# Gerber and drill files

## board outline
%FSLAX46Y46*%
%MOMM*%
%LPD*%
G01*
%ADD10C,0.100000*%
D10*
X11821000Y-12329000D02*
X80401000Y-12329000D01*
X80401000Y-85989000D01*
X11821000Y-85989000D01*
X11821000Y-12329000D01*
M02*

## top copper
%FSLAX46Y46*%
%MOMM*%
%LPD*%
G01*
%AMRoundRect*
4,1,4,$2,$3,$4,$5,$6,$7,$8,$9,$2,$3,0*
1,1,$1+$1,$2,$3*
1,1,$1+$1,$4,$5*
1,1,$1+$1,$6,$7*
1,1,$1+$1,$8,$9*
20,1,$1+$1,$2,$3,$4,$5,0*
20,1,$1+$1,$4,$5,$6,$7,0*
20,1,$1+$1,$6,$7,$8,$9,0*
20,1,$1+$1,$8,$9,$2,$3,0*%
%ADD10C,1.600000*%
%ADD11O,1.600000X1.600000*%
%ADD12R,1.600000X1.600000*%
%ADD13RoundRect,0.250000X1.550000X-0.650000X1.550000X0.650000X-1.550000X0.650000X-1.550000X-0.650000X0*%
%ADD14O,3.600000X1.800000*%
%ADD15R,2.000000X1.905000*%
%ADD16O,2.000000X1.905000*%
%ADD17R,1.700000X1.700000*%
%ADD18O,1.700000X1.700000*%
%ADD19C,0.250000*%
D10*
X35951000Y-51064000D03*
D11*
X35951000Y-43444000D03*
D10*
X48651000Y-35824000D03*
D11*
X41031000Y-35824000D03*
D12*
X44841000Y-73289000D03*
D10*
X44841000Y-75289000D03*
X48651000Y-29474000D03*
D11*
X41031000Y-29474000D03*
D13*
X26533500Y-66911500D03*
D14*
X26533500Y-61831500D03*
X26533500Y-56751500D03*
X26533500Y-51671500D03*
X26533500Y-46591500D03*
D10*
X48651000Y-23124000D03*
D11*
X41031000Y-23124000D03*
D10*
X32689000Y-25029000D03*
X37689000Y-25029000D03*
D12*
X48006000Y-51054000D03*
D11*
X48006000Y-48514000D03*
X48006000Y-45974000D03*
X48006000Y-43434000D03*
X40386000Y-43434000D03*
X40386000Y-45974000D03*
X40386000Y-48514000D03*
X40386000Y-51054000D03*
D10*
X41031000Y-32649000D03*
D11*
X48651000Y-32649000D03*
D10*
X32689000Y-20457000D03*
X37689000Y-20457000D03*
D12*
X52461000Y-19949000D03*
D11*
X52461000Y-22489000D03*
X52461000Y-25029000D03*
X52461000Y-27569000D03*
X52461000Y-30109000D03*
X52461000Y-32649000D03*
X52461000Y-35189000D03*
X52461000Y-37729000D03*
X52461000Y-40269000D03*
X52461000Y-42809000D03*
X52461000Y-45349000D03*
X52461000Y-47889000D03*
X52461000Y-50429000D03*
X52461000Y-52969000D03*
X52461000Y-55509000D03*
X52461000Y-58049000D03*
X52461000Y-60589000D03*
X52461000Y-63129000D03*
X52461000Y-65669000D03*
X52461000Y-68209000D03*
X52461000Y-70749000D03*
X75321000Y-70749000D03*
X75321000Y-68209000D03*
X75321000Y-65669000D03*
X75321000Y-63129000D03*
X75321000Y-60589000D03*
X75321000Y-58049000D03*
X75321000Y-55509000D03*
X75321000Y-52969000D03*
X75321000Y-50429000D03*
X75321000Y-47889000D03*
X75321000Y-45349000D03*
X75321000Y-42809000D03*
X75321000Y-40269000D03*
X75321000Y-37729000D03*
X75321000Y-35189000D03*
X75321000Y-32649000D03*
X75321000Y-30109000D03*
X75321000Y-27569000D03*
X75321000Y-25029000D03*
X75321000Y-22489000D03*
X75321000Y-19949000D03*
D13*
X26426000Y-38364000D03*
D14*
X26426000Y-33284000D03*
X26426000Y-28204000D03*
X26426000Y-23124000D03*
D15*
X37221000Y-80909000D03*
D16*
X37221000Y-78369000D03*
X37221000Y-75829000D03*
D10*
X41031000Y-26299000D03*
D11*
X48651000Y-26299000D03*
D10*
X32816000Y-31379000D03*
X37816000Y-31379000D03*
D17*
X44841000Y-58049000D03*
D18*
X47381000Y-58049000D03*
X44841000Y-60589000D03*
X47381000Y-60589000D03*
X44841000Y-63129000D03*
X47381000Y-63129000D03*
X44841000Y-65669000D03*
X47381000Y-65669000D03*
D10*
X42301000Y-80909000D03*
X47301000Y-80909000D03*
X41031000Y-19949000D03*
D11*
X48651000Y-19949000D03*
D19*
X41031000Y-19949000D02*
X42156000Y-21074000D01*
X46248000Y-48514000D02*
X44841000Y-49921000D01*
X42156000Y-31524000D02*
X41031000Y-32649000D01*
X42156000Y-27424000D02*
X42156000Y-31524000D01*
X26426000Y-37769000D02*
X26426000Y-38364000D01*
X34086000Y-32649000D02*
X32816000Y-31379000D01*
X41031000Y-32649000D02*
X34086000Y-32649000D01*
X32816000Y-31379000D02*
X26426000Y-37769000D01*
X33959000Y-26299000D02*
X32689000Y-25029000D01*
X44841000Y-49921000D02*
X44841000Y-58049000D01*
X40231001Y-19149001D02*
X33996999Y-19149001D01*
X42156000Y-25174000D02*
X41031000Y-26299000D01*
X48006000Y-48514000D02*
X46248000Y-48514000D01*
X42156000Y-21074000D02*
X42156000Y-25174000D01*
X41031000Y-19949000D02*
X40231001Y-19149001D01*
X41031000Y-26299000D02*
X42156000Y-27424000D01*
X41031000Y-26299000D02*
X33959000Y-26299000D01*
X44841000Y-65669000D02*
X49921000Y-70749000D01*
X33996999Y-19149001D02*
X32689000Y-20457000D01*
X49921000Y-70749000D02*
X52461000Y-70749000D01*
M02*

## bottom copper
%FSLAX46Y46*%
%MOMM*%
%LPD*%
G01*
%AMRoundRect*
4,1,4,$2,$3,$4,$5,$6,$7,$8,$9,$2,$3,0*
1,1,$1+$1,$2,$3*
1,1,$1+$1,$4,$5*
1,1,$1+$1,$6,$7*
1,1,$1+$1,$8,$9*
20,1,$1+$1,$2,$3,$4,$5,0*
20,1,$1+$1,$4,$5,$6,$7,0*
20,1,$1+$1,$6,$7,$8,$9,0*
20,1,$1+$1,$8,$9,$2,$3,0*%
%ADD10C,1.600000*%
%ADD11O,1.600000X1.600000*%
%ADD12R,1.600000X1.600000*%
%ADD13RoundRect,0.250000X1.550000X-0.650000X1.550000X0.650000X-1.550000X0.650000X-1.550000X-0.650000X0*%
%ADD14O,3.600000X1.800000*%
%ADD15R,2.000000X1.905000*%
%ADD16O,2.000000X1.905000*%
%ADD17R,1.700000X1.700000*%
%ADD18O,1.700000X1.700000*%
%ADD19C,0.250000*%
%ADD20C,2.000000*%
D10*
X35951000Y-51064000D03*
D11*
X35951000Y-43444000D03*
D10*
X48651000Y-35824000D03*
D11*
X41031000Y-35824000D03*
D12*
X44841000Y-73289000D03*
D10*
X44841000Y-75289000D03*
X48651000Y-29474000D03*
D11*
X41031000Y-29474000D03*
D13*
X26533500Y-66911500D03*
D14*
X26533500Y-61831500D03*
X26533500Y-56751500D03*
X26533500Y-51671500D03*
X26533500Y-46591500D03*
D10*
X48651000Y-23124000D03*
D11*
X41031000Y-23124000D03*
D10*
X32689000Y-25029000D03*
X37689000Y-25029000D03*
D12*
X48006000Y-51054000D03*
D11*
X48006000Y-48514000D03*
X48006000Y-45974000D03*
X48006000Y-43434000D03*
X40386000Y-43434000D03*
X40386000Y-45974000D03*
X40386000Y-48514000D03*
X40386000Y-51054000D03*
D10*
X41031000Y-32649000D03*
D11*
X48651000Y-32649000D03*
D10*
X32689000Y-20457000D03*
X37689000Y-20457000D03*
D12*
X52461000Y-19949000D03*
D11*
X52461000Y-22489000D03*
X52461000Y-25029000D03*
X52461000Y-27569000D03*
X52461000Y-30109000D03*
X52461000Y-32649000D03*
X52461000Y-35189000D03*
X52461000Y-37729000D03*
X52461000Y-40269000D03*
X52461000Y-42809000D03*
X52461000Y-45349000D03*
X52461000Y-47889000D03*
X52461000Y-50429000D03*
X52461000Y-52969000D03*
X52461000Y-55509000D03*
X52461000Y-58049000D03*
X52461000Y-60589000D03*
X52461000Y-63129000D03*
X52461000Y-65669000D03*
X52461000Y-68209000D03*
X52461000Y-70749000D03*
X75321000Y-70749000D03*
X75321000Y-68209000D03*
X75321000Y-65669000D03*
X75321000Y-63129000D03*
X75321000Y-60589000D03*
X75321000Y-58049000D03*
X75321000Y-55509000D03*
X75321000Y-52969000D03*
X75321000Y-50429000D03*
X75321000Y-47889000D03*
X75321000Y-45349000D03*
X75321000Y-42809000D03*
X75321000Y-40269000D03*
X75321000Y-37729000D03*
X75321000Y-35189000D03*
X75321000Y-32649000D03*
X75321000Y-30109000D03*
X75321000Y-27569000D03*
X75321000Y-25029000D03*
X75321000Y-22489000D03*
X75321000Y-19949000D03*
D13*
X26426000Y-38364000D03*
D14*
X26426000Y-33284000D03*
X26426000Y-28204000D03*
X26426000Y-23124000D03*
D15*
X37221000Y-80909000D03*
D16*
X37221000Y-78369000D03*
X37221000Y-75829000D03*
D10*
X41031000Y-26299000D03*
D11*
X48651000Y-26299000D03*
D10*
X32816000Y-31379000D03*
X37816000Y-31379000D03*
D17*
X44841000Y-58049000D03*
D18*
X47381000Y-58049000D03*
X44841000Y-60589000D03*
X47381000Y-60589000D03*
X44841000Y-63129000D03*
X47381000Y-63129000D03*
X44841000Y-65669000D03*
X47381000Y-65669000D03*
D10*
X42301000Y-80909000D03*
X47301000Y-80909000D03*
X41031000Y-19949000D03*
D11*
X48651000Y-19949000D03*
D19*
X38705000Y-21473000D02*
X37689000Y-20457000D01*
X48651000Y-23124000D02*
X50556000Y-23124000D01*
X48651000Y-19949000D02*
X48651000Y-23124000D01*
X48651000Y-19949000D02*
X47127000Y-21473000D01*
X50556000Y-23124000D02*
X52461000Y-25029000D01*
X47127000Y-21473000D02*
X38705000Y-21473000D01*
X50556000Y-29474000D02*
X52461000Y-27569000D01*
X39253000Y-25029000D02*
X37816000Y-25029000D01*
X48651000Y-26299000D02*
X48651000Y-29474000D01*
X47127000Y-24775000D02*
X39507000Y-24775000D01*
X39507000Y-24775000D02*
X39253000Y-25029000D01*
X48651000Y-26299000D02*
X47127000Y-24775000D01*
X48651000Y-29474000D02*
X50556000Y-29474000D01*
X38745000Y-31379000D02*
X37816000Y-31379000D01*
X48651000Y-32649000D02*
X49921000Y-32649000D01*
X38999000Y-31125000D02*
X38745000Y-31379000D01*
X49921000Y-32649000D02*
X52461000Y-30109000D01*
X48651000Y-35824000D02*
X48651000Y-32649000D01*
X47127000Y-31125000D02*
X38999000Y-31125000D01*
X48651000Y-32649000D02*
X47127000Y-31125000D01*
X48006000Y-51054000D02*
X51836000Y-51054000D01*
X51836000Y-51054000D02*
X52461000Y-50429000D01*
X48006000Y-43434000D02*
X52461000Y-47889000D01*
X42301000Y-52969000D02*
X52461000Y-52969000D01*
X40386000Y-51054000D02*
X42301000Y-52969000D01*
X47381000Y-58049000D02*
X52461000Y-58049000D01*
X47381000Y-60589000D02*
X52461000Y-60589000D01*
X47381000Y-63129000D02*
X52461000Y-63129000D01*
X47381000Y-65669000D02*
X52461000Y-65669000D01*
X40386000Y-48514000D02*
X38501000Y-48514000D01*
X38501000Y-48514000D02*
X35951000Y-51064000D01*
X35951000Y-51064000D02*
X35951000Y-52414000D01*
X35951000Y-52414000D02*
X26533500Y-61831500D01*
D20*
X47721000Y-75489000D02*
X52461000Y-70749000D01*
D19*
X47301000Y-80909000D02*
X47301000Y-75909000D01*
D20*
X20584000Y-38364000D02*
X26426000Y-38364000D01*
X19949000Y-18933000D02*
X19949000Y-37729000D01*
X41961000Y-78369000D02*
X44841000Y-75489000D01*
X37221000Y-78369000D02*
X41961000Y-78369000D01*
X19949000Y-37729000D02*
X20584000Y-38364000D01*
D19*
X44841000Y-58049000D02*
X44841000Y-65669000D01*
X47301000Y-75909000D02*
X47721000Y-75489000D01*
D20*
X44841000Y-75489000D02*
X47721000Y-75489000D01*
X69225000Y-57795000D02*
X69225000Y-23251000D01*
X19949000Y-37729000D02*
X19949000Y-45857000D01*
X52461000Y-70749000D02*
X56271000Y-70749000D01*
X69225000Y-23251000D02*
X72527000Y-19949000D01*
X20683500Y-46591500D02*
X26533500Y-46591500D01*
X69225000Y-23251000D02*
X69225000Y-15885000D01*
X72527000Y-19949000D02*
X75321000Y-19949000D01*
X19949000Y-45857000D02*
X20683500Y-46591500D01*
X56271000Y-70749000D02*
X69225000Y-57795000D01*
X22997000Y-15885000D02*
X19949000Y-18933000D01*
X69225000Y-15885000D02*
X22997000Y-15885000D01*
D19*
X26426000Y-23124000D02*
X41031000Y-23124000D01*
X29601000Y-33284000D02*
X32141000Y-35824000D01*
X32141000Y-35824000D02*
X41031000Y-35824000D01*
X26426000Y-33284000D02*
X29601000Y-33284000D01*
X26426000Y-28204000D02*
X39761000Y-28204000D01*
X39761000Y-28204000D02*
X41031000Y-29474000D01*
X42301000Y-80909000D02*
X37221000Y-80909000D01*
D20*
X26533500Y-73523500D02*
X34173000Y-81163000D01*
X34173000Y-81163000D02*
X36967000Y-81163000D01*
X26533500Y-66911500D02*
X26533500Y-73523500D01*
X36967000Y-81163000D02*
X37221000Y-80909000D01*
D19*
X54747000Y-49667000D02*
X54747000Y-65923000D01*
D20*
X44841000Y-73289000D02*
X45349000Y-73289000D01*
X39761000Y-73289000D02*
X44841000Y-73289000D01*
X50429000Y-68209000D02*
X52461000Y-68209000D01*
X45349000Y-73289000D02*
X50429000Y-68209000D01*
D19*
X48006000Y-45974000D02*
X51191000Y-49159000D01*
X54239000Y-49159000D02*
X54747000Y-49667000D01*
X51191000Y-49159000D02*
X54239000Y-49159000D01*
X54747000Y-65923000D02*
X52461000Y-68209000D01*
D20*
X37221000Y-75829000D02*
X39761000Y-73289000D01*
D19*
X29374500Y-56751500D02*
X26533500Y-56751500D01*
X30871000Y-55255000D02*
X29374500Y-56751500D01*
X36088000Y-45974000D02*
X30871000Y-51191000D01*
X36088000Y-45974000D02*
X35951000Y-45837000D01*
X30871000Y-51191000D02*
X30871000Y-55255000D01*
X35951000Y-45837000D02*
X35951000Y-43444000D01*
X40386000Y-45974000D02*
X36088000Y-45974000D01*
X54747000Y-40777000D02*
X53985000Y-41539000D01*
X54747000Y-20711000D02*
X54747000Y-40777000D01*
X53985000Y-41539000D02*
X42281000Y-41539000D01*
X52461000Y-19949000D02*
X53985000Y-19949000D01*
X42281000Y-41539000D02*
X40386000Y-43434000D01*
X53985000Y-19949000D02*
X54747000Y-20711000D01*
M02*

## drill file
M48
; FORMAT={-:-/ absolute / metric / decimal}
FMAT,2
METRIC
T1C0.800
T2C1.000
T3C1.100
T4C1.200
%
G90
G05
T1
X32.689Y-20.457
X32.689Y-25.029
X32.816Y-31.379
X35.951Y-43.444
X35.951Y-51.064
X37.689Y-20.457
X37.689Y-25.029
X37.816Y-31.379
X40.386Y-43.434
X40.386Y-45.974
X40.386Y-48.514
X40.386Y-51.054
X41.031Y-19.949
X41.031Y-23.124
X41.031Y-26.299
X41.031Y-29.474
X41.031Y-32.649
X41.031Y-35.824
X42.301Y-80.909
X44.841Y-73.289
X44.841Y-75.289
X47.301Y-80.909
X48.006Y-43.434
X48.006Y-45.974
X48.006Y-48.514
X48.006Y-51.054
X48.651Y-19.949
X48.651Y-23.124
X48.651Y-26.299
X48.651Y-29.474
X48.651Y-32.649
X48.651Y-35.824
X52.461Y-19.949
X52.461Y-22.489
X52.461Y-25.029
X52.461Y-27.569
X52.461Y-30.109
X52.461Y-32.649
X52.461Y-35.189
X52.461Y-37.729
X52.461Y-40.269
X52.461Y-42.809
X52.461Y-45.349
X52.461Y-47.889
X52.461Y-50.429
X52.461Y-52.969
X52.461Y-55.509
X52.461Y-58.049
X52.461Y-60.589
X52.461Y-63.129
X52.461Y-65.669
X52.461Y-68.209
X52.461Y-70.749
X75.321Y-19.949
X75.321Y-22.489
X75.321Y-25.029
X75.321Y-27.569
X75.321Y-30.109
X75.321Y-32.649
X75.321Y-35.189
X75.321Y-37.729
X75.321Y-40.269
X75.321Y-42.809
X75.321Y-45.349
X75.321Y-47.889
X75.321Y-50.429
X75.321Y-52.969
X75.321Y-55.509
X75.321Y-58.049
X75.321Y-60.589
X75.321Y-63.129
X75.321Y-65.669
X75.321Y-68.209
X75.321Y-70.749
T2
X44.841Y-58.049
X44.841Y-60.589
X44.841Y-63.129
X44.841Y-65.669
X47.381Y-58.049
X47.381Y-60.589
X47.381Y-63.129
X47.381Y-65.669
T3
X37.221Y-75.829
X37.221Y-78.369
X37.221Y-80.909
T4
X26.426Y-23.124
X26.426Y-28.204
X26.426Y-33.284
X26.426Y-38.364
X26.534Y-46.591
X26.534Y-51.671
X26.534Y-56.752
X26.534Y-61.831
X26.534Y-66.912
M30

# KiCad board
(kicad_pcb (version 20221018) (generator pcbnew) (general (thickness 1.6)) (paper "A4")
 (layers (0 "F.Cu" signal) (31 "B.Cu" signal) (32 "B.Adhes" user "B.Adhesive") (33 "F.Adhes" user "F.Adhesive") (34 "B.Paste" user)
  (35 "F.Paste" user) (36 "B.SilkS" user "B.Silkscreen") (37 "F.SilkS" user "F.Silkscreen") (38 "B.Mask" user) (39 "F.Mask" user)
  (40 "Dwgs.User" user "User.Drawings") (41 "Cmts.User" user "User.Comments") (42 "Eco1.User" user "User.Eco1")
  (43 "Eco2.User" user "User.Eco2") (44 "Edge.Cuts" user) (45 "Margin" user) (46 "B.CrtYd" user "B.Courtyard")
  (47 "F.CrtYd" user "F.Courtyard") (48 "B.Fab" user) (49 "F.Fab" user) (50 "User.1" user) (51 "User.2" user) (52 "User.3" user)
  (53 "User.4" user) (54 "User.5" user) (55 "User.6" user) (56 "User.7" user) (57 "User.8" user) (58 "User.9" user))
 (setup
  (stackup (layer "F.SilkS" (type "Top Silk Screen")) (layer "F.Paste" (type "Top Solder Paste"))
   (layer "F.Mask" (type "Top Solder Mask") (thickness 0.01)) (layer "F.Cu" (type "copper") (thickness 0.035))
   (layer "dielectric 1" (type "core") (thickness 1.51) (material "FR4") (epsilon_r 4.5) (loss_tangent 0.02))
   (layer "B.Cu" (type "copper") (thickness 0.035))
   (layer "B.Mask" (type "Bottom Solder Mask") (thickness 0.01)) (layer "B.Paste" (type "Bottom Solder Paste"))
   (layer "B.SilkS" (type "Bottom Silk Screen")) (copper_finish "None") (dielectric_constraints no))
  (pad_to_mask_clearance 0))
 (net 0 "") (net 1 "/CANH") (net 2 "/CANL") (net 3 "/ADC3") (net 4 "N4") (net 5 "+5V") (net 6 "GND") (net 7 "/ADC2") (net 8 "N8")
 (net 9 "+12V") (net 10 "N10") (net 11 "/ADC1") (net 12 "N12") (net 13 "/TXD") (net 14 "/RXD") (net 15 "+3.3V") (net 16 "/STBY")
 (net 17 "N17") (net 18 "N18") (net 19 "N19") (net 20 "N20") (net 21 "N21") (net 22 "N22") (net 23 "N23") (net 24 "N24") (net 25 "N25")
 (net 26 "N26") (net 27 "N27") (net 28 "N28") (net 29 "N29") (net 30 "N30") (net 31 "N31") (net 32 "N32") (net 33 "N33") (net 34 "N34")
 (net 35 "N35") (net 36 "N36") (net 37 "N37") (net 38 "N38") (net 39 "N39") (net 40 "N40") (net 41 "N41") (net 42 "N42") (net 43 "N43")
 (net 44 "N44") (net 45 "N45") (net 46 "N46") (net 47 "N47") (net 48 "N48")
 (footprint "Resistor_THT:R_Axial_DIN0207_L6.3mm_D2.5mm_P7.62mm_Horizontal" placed (layer "F.Cu") (at 35.951 51.064 90)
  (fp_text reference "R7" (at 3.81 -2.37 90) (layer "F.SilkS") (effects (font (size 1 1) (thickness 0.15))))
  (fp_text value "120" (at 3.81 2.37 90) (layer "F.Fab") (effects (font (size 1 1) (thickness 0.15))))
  (pad "1" thru_hole circle (at 0 0 90) (size 1.6 1.6) (drill 0.8) (layers "*.Cu" "*.Mask") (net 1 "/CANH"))
  (pad "2" thru_hole oval (at 7.62 0 90) (size 1.6 1.6) (drill 0.8) (layers "*.Cu" "*.Mask") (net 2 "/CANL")))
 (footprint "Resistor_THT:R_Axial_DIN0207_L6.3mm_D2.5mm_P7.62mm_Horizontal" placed (layer "F.Cu") (at 48.651 35.824 180)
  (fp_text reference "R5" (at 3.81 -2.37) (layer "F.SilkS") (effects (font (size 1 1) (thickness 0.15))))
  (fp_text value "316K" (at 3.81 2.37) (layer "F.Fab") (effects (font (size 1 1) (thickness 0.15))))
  (pad "1" thru_hole circle (at 0 0 180) (size 1.6 1.6) (drill 0.8) (layers "*.Cu" "*.Mask") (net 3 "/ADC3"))
  (pad "2" thru_hole oval (at 7.62 0 180) (size 1.6 1.6) (drill 0.8) (layers "*.Cu" "*.Mask") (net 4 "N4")))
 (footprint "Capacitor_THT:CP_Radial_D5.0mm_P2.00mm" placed (layer "F.Cu") (at 44.841 73.289 -90)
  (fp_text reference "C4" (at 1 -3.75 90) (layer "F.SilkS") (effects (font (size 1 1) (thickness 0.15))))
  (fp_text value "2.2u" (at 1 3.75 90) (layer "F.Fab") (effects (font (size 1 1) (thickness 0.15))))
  (pad "1" thru_hole rect (at 0 0 270) (size 1.6 1.6) (drill 0.8) (layers "*.Cu" "*.Mask") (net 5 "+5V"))
  (pad "2" thru_hole circle (at 2 0 270) (size 1.6 1.6) (drill 0.8) (layers "*.Cu" "*.Mask") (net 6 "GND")))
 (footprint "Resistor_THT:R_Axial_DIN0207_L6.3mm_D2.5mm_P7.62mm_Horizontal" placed (layer "F.Cu") (at 48.651 29.474 180)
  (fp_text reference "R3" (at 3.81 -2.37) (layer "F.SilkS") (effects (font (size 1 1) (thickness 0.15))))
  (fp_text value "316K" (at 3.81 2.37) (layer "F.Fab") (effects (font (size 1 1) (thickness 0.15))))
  (pad "1" thru_hole circle (at 0 0 180) (size 1.6 1.6) (drill 0.8) (layers "*.Cu" "*.Mask") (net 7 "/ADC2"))
  (pad "2" thru_hole oval (at 7.62 0 180) (size 1.6 1.6) (drill 0.8) (layers "*.Cu" "*.Mask") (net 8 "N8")))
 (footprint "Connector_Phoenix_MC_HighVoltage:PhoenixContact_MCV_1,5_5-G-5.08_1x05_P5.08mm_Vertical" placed (layer "F.Cu")
  (at 26.5335 66.9115 90)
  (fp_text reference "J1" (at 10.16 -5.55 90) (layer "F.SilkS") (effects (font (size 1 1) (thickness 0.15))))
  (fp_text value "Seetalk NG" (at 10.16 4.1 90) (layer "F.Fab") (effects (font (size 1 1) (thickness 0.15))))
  (pad "1" thru_hole roundrect (at 0 0 90) (size 1.8 3.6) (drill 1.2) (layers "*.Cu" "*.Mask") (roundrect_rratio 0.138889) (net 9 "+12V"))
  (pad "2" thru_hole oval (at 5.08 0 90) (size 1.8 3.6) (drill 1.2) (layers "*.Cu" "*.Mask") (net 1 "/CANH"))
  (pad "3" thru_hole oval (at 10.16 0 90) (size 1.8 3.6) (drill 1.2) (layers "*.Cu" "*.Mask") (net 2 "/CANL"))
  (pad "4" thru_hole oval (at 15.24 0 90) (size 1.8 3.6) (drill 1.2) (layers "*.Cu" "*.Mask") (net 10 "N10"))
  (pad "5" thru_hole oval (at 20.32 0 90) (size 1.8 3.6) (drill 1.2) (layers "*.Cu" "*.Mask") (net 6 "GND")))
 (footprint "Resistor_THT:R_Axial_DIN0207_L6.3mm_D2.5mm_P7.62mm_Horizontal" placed (layer "F.Cu") (at 48.651 23.124 180)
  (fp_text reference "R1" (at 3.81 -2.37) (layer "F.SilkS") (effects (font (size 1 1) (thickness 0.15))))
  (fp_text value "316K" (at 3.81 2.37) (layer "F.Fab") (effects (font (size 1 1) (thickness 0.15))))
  (pad "1" thru_hole circle (at 0 0 180) (size 1.6 1.6) (drill 0.8) (layers "*.Cu" "*.Mask") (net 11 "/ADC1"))
  (pad "2" thru_hole oval (at 7.62 0 180) (size 1.6 1.6) (drill 0.8) (layers "*.Cu" "*.Mask") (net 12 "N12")))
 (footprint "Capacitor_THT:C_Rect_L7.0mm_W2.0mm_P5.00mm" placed (layer "F.Cu") (at 32.689 25.029)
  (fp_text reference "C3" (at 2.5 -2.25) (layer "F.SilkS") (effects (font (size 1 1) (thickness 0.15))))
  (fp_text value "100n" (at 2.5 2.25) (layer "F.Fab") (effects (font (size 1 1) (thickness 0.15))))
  (pad "1" thru_hole circle (at 0 0) (size 1.6 1.6) (drill 0.8) (layers "*.Cu" "*.Mask") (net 6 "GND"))
  (pad "2" thru_hole circle (at 5 0) (size 1.6 1.6) (drill 0.8) (layers "*.Cu" "*.Mask") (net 7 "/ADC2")))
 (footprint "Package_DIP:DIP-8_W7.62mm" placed (layer "F.Cu") (at 48.006 51.054 180)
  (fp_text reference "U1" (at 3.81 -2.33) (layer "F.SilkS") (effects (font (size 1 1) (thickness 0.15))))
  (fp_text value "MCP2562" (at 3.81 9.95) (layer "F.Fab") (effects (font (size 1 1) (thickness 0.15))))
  (pad "1" thru_hole rect (at 0 0 180) (size 1.6 1.6) (drill 0.8) (layers "*.Cu" "*.Mask") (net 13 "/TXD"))
  (pad "2" thru_hole oval (at 0 2.54 180) (size 1.6 1.6) (drill 0.8) (layers "*.Cu" "*.Mask") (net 6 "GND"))
  (pad "3" thru_hole oval (at 0 5.08 180) (size 1.6 1.6) (drill 0.8) (layers "*.Cu" "*.Mask") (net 5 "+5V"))
  (pad "4" thru_hole oval (at 0 7.62 180) (size 1.6 1.6) (drill 0.8) (layers "*.Cu" "*.Mask") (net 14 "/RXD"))
  (pad "5" thru_hole oval (at 7.62 7.62 180) (size 1.6 1.6) (drill 0.8) (layers "*.Cu" "*.Mask") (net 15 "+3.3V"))
  (pad "6" thru_hole oval (at 7.62 5.08 180) (size 1.6 1.6) (drill 0.8) (layers "*.Cu" "*.Mask") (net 2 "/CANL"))
  (pad "7" thru_hole oval (at 7.62 2.54 180) (size 1.6 1.6) (drill 0.8) (layers "*.Cu" "*.Mask") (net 1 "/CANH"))
  (pad "8" thru_hole oval (at 7.62 0 180) (size 1.6 1.6) (drill 0.8) (layers "*.Cu" "*.Mask") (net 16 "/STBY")))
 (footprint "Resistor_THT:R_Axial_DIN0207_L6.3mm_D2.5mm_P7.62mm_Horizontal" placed (layer "F.Cu") (at 41.031 32.649)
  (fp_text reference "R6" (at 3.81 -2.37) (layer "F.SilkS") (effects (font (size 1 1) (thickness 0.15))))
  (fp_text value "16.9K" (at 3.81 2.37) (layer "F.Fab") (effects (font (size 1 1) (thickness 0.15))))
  (pad "1" thru_hole circle (at 0 0) (size 1.6 1.6) (drill 0.8) (layers "*.Cu" "*.Mask") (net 6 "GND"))
  (pad "2" thru_hole oval (at 7.62 0) (size 1.6 1.6) (drill 0.8) (layers "*.Cu" "*.Mask") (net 3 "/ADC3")))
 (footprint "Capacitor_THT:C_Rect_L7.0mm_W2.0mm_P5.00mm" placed (layer "F.Cu") (at 32.689 20.457)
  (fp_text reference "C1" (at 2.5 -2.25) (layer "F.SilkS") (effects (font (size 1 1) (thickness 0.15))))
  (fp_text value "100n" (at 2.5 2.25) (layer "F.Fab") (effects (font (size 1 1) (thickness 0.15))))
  (pad "1" thru_hole circle (at 0 0) (size 1.6 1.6) (drill 0.8) (layers "*.Cu" "*.Mask") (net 6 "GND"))
  (pad "2" thru_hole circle (at 5 0) (size 1.6 1.6) (drill 0.8) (layers "*.Cu" "*.Mask") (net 11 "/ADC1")))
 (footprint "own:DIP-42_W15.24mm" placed (layer "F.Cu") (at 52.461 19.949)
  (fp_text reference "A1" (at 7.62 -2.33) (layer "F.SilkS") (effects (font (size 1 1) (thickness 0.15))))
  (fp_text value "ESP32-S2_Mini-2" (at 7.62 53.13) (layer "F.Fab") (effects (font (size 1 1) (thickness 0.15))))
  (pad "1" thru_hole rect (at 0 0) (size 1.6 1.6) (drill 0.8) (layers "*.Cu" "*.Mask") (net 15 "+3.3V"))
  (pad "2" thru_hole oval (at 0 2.54) (size 1.6 1.6) (drill 0.8) (layers "*.Cu" "*.Mask") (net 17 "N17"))
  (pad "3" thru_hole oval (at 0 5.08) (size 1.6 1.6) (drill 0.8) (layers "*.Cu" "*.Mask") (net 11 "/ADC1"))
  (pad "4" thru_hole oval (at 0 7.62) (size 1.6 1.6) (drill 0.8) (layers "*.Cu" "*.Mask") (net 7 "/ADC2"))
  (pad "5" thru_hole oval (at 0 10.16) (size 1.6 1.6) (drill 0.8) (layers "*.Cu" "*.Mask") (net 3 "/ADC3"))
  (pad "6" thru_hole oval (at 0 12.7) (size 1.6 1.6) (drill 0.8) (layers "*.Cu" "*.Mask") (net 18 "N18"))
  (pad "7" thru_hole oval (at 0 15.24) (size 1.6 1.6) (drill 0.8) (layers "*.Cu" "*.Mask") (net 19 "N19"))
  (pad "8" thru_hole oval (at 0 17.78) (size 1.6 1.6) (drill 0.8) (layers "*.Cu" "*.Mask") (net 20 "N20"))
  (pad "9" thru_hole oval (at 0 20.32) (size 1.6 1.6) (drill 0.8) (layers "*.Cu" "*.Mask") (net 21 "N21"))
  (pad "10" thru_hole oval (at 0 22.86) (size 1.6 1.6) (drill 0.8) (layers "*.Cu" "*.Mask") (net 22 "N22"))
  (pad "11" thru_hole oval (at 0 25.4) (size 1.6 1.6) (drill 0.8) (layers "*.Cu" "*.Mask") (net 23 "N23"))
  (pad "12" thru_hole oval (at 0 27.94) (size 1.6 1.6) (drill 0.8) (layers "*.Cu" "*.Mask") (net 14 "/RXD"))
  (pad "13" thru_hole oval (at 0 30.48) (size 1.6 1.6) (drill 0.8) (layers "*.Cu" "*.Mask") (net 13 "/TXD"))
  (pad "14" thru_hole oval (at 0 33.02) (size 1.6 1.6) (drill 0.8) (layers "*.Cu" "*.Mask") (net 16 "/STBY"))
  (pad "15" thru_hole oval (at 0 35.56) (size 1.6 1.6) (drill 0.8) (layers "*.Cu" "*.Mask") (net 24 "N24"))
  (pad "16" thru_hole oval (at 0 38.1) (size 1.6 1.6) (drill 0.8) (layers "*.Cu" "*.Mask") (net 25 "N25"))
  (pad "17" thru_hole oval (at 0 40.64) (size 1.6 1.6) (drill 0.8) (layers "*.Cu" "*.Mask") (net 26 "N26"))
  (pad "18" thru_hole oval (at 0 43.18) (size 1.6 1.6) (drill 0.8) (layers "*.Cu" "*.Mask") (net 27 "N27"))
  (pad "19" thru_hole oval (at 0 45.72) (size 1.6 1.6) (drill 0.8) (layers "*.Cu" "*.Mask") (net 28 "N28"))
  (pad "20" thru_hole oval (at 0 48.26) (size 1.6 1.6) (drill 0.8) (layers "*.Cu" "*.Mask") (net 5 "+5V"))
  (pad "21" thru_hole oval (at 0 50.8) (size 1.6 1.6) (drill 0.8) (layers "*.Cu" "*.Mask") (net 6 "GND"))
  (pad "22" thru_hole oval (at 22.86 50.8) (size 1.6 1.6) (drill 0.8) (layers "*.Cu" "*.Mask") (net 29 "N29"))
  (pad "23" thru_hole oval (at 22.86 48.26) (size 1.6 1.6) (drill 0.8) (layers "*.Cu" "*.Mask") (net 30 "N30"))
  (pad "24" thru_hole oval (at 22.86 45.72) (size 1.6 1.6) (drill 0.8) (layers "*.Cu" "*.Mask") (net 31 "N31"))
  (pad "25" thru_hole oval (at 22.86 43.18) (size 1.6 1.6) (drill 0.8) (layers "*.Cu" "*.Mask") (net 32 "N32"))
  (pad "26" thru_hole oval (at 22.86 40.64) (size 1.6 1.6) (drill 0.8) (layers "*.Cu" "*.Mask") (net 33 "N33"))
  (pad "27" thru_hole oval (at 22.86 38.1) (size 1.6 1.6) (drill 0.8) (layers "*.Cu" "*.Mask") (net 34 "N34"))
  (pad "28" thru_hole oval (at 22.86 35.56) (size 1.6 1.6) (drill 0.8) (layers "*.Cu" "*.Mask") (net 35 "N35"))
  (pad "29" thru_hole oval (at 22.86 33.02) (size 1.6 1.6) (drill 0.8) (layers "*.Cu" "*.Mask") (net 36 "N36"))
  (pad "30" thru_hole oval (at 22.86 30.48) (size 1.6 1.6) (drill 0.8) (layers "*.Cu" "*.Mask") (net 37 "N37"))
  (pad "31" thru_hole oval (at 22.86 27.94) (size 1.6 1.6) (drill 0.8) (layers "*.Cu" "*.Mask") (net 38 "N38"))
  (pad "32" thru_hole oval (at 22.86 25.4) (size 1.6 1.6) (drill 0.8) (layers "*.Cu" "*.Mask") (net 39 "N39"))
  (pad "33" thru_hole oval (at 22.86 22.86) (size 1.6 1.6) (drill 0.8) (layers "*.Cu" "*.Mask") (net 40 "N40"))
  (pad "34" thru_hole oval (at 22.86 20.32) (size 1.6 1.6) (drill 0.8) (layers "*.Cu" "*.Mask") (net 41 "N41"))
  (pad "35" thru_hole oval (at 22.86 17.78) (size 1.6 1.6) (drill 0.8) (layers "*.Cu" "*.Mask") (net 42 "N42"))
  (pad "36" thru_hole oval (at 22.86 15.24) (size 1.6 1.6) (drill 0.8) (layers "*.Cu" "*.Mask") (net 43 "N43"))
  (pad "37" thru_hole oval (at 22.86 12.7) (size 1.6 1.6) (drill 0.8) (layers "*.Cu" "*.Mask") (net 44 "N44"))
  (pad "38" thru_hole oval (at 22.86 10.16) (size 1.6 1.6) (drill 0.8) (layers "*.Cu" "*.Mask") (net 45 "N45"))
  (pad "39" thru_hole oval (at 22.86 7.62) (size 1.6 1.6) (drill 0.8) (layers "*.Cu" "*.Mask") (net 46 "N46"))
  (pad "40" thru_hole oval (at 22.86 5.08) (size 1.6 1.6) (drill 0.8) (layers "*.Cu" "*.Mask") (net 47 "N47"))
  (pad "41" thru_hole oval (at 22.86 2.54) (size 1.6 1.6) (drill 0.8) (layers "*.Cu" "*.Mask") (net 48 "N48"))
  (pad "42" thru_hole oval (at 22.86 0) (size 1.6 1.6) (drill 0.8) (layers "*.Cu" "*.Mask") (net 6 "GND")))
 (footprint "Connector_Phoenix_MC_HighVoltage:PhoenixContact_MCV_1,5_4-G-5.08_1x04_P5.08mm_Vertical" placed (layer "F.Cu")
  (at 26.426 38.364 90)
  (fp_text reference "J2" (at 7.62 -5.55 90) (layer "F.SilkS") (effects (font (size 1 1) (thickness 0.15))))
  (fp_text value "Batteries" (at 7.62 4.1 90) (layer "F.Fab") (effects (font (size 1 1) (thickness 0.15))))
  (pad "1" thru_hole roundrect (at 0 0 90) (size 1.8 3.6) (drill 1.2) (layers "*.Cu" "*.Mask") (roundrect_rratio 0.138889) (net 6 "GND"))
  (pad "2" thru_hole oval (at 5.08 0 90) (size 1.8 3.6) (drill 1.2) (layers "*.Cu" "*.Mask") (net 4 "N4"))
  (pad "3" thru_hole oval (at 10.16 0 90) (size 1.8 3.6) (drill 1.2) (layers "*.Cu" "*.Mask") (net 8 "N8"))
  (pad "4" thru_hole oval (at 15.24 0 90) (size 1.8 3.6) (drill 1.2) (layers "*.Cu" "*.Mask") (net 12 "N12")))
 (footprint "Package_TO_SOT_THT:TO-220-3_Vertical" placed (layer "F.Cu") (at 37.221 80.909 90)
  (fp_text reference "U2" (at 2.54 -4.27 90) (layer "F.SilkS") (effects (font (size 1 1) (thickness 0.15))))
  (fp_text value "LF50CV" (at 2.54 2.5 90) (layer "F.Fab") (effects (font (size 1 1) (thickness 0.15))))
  (pad "1" thru_hole rect (at 0 0 90) (size 1.905 2) (drill 1.1) (layers "*.Cu" "*.Mask") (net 9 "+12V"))
  (pad "2" thru_hole oval (at 2.54 0 90) (size 1.905 2) (drill 1.1) (layers "*.Cu" "*.Mask") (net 6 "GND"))
  (pad "3" thru_hole oval (at 5.08 0 90) (size 1.905 2) (drill 1.1) (layers "*.Cu" "*.Mask") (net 5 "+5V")))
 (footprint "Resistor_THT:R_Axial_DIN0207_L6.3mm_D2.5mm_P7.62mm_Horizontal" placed (layer "F.Cu") (at 41.031 26.299)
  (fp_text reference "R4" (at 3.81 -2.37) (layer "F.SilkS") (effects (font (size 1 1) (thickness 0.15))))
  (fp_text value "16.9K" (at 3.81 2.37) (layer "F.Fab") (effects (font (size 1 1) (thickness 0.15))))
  (pad "1" thru_hole circle (at 0 0) (size 1.6 1.6) (drill 0.8) (layers "*.Cu" "*.Mask") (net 6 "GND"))
  (pad "2" thru_hole oval (at 7.62 0) (size 1.6 1.6) (drill 0.8) (layers "*.Cu" "*.Mask") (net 7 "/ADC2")))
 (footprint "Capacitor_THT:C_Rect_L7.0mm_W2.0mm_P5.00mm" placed (layer "F.Cu") (at 32.816 31.379)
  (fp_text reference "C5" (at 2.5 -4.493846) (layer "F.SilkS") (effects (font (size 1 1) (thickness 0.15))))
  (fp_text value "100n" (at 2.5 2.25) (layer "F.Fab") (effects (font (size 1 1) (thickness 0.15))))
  (pad "1" thru_hole circle (at 0 0) (size 1.6 1.6) (drill 0.8) (layers "*.Cu" "*.Mask") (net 6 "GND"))
  (pad "2" thru_hole circle (at 5 0) (size 1.6 1.6) (drill 0.8) (layers "*.Cu" "*.Mask") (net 3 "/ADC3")))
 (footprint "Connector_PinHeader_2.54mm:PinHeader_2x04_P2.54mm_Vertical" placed (layer "F.Cu") (at 44.841 58.049)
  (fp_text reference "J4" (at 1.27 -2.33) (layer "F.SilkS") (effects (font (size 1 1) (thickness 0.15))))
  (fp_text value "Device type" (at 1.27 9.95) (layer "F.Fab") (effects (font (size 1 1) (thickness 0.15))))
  (pad "1" thru_hole rect (at 0 0) (size 1.7 1.7) (drill 1) (layers "*.Cu" "*.Mask") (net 6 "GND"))
  (pad "2" thru_hole oval (at 2.54 0) (size 1.7 1.7) (drill 1) (layers "*.Cu" "*.Mask") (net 25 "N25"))
  (pad "3" thru_hole oval (at 0 2.54) (size 1.7 1.7) (drill 1) (layers "*.Cu" "*.Mask") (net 6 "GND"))
  (pad "4" thru_hole oval (at 2.54 2.54) (size 1.7 1.7) (drill 1) (layers "*.Cu" "*.Mask") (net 26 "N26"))
  (pad "5" thru_hole oval (at 0 5.08) (size 1.7 1.7) (drill 1) (layers "*.Cu" "*.Mask") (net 6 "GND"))
  (pad "6" thru_hole oval (at 2.54 5.08) (size 1.7 1.7) (drill 1) (layers "*.Cu" "*.Mask") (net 27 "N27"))
  (pad "7" thru_hole oval (at 0 7.62) (size 1.7 1.7) (drill 1) (layers "*.Cu" "*.Mask") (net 6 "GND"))
  (pad "8" thru_hole oval (at 2.54 7.62) (size 1.7 1.7) (drill 1) (layers "*.Cu" "*.Mask") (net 28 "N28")))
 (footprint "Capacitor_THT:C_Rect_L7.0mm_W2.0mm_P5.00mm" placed (layer "F.Cu") (at 42.301 80.909)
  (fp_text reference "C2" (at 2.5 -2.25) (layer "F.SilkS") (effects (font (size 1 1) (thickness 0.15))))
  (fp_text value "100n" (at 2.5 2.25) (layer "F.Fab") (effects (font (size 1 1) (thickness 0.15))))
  (pad "1" thru_hole circle (at 0 0) (size 1.6 1.6) (drill 0.8) (layers "*.Cu" "*.Mask") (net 9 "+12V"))
  (pad "2" thru_hole circle (at 5 0) (size 1.6 1.6) (drill 0.8) (layers "*.Cu" "*.Mask") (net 6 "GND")))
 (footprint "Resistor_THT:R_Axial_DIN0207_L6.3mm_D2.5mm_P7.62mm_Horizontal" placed (layer "F.Cu") (at 41.031 19.949)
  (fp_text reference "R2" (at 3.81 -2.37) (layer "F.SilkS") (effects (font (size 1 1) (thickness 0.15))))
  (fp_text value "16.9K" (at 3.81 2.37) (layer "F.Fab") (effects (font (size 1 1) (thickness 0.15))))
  (pad "1" thru_hole circle (at 0 0) (size 1.6 1.6) (drill 0.8) (layers "*.Cu" "*.Mask") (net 6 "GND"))
  (pad "2" thru_hole oval (at 7.62 0) (size 1.6 1.6) (drill 0.8) (layers "*.Cu" "*.Mask") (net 11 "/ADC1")))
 (gr_rect (start 11.821 12.329) (end 80.401 85.989) (stroke (width 0.1) (type default)) (fill none) (layer "Edge.Cuts"))
 (segment (start 38.705 21.473) (end 37.689 20.457) (width 0.25) (layer "B.Cu") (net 11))
 (segment (start 48.651 23.124) (end 50.556 23.124) (width 0.25) (layer "B.Cu") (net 11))
 (segment (start 48.651 19.949) (end 48.651 23.124) (width 0.25) (layer "B.Cu") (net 11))
 (segment (start 48.651 19.949) (end 47.127 21.473) (width 0.25) (layer "B.Cu") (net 11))
 (segment (start 50.556 23.124) (end 52.461 25.029) (width 0.25) (layer "B.Cu") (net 11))
 (segment (start 47.127 21.473) (end 38.705 21.473) (width 0.25) (layer "B.Cu") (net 11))
 (segment (start 50.556 29.474) (end 52.461 27.569) (width 0.25) (layer "B.Cu") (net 7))
 (segment (start 39.253 25.029) (end 37.816 25.029) (width 0.25) (layer "B.Cu") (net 7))
 (segment (start 48.651 26.299) (end 48.651 29.474) (width 0.25) (layer "B.Cu") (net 7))
 (segment (start 47.127 24.775) (end 39.507 24.775) (width 0.25) (layer "B.Cu") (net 7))
 (segment (start 39.507 24.775) (end 39.253 25.029) (width 0.25) (layer "B.Cu") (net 7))
 (segment (start 48.651 26.299) (end 47.127 24.775) (width 0.25) (layer "B.Cu") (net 7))
 (segment (start 48.651 29.474) (end 50.556 29.474) (width 0.25) (layer "B.Cu") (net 7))
 (segment (start 38.745 31.379) (end 37.816 31.379) (width 0.25) (layer "B.Cu") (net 3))
 (segment (start 48.651 32.649) (end 49.921 32.649) (width 0.25) (layer "B.Cu") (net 3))
 (segment (start 38.999 31.125) (end 38.745 31.379) (width 0.25) (layer "B.Cu") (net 3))
 (segment (start 49.921 32.649) (end 52.461 30.109) (width 0.25) (layer "B.Cu") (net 3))
 (segment (start 48.651 35.824) (end 48.651 32.649) (width 0.25) (layer "B.Cu") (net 3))
 (segment (start 47.127 31.125) (end 38.999 31.125) (width 0.25) (layer "B.Cu") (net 3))
 (segment (start 48.651 32.649) (end 47.127 31.125) (width 0.25) (layer "B.Cu") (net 3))
 (segment (start 48.006 51.054) (end 51.836 51.054) (width 0.25) (layer "B.Cu") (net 13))
 (segment (start 51.836 51.054) (end 52.461 50.429) (width 0.25) (layer "B.Cu") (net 13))
 (segment (start 48.006 43.434) (end 52.461 47.889) (width 0.25) (layer "B.Cu") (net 14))
 (segment (start 42.301 52.969) (end 52.461 52.969) (width 0.25) (layer "B.Cu") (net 16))
 (segment (start 40.386 51.054) (end 42.301 52.969) (width 0.25) (layer "B.Cu") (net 16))
 (segment (start 47.381 58.049) (end 52.461 58.049) (width 0.25) (layer "B.Cu") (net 25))
 (segment (start 47.381 60.589) (end 52.461 60.589) (width 0.25) (layer "B.Cu") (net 26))
 (segment (start 47.381 63.129) (end 52.461 63.129) (width 0.25) (layer "B.Cu") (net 27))
 (segment (start 47.381 65.669) (end 52.461 65.669) (width 0.25) (layer "B.Cu") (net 28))
 (segment (start 40.386 48.514) (end 38.501 48.514) (width 0.25) (layer "B.Cu") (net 1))
 (segment (start 38.501 48.514) (end 35.951 51.064) (width 0.25) (layer "B.Cu") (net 1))
 (segment (start 35.951 51.064) (end 35.951 52.414) (width 0.25) (layer "B.Cu") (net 1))
 (segment (start 35.951 52.414) (end 26.5335 61.8315) (width 0.25) (layer "B.Cu") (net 1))
 (segment (start 41.031 19.949) (end 42.156 21.074) (width 0.25) (layer "F.Cu") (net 6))
 (segment (start 46.248 48.514) (end 44.841 49.921) (width 0.25) (layer "F.Cu") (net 6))
 (segment (start 42.156 31.524) (end 41.031 32.649) (width 0.25) (layer "F.Cu") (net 6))
 (segment (start 42.156 27.424) (end 42.156 31.524) (width 0.25) (layer "F.Cu") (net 6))
 (segment (start 26.426 37.769) (end 26.426 38.364) (width 0.25) (layer "F.Cu") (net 6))
 (segment (start 34.086 32.649) (end 32.816 31.379) (width 0.25) (layer "F.Cu") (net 6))
 (segment (start 41.031 32.649) (end 34.086 32.649) (width 0.25) (layer "F.Cu") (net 6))
 (segment (start 32.816 31.379) (end 26.426 37.769) (width 0.25) (layer "F.Cu") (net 6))
 (segment (start 33.959 26.299) (end 32.689 25.029) (width 0.25) (layer "F.Cu") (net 6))
 (segment (start 44.841 49.921) (end 44.841 58.049) (width 0.25) (layer "F.Cu") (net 6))
 (segment (start 40.231001 19.149001) (end 33.996999 19.149001) (width 0.25) (layer "F.Cu") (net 6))
 (segment (start 42.156 25.174) (end 41.031 26.299) (width 0.25) (layer "F.Cu") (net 6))
 (segment (start 48.006 48.514) (end 46.248 48.514) (width 0.25) (layer "F.Cu") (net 6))
 (segment (start 42.156 21.074) (end 42.156 25.174) (width 0.25) (layer "F.Cu") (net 6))
 (segment (start 41.031 19.949) (end 40.231001 19.149001) (width 0.25) (layer "F.Cu") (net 6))
 (segment (start 41.031 26.299) (end 42.156 27.424) (width 0.25) (layer "F.Cu") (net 6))
 (segment (start 41.031 26.299) (end 33.959 26.299) (width 0.25) (layer "F.Cu") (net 6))
 (segment (start 44.841 65.669) (end 49.921 70.749) (width 0.25) (layer "F.Cu") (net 6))
 (segment (start 33.996999 19.149001) (end 32.689 20.457) (width 0.25) (layer "F.Cu") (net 6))
 (segment (start 49.921 70.749) (end 52.461 70.749) (width 0.25) (layer "F.Cu") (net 6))
 (segment (start 47.721 75.489) (end 52.461 70.749) (width 2) (layer "B.Cu") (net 6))
 (segment (start 47.301 80.909) (end 47.301 75.909) (width 0.25) (layer "B.Cu") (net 6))
 (segment (start 20.584 38.364) (end 26.426 38.364) (width 2) (layer "B.Cu") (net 6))
 (segment (start 19.949 18.933) (end 19.949 37.729) (width 2) (layer "B.Cu") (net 6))
 (segment (start 41.961 78.369) (end 44.841 75.489) (width 2) (layer "B.Cu") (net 6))
 (segment (start 37.221 78.369) (end 41.961 78.369) (width 2) (layer "B.Cu") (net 6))
 (segment (start 19.949 37.729) (end 20.584 38.364) (width 2) (layer "B.Cu") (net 6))
 (segment (start 44.841 58.049) (end 44.841 65.669) (width 0.25) (layer "B.Cu") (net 6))
 (segment (start 47.301 75.909) (end 47.721 75.489) (width 0.25) (layer "B.Cu") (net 6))
 (segment (start 44.841 75.489) (end 47.721 75.489) (width 2) (layer "B.Cu") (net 6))
 (segment (start 69.225 57.795) (end 69.225 23.251) (width 2) (layer "B.Cu") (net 6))
 (segment (start 19.949 37.729) (end 19.949 45.857) (width 2) (layer "B.Cu") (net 6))
 (segment (start 52.461 70.749) (end 56.271 70.749) (width 2) (layer "B.Cu") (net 6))
 (segment (start 69.225 23.251) (end 72.527 19.949) (width 2) (layer "B.Cu") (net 6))
 (segment (start 20.6835 46.5915) (end 26.5335 46.5915) (width 2) (layer "B.Cu") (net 6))
 (segment (start 69.225 23.251) (end 69.225 15.885) (width 2) (layer "B.Cu") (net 6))
 (segment (start 72.527 19.949) (end 75.321 19.949) (width 2) (layer "B.Cu") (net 6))
 (segment (start 19.949 45.857) (end 20.6835 46.5915) (width 2) (layer "B.Cu") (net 6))
 (segment (start 56.271 70.749) (end 69.225 57.795) (width 2) (layer "B.Cu") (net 6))
 (segment (start 22.997 15.885) (end 19.949 18.933) (width 2) (layer "B.Cu") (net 6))
 (segment (start 69.225 15.885) (end 22.997 15.885) (width 2) (layer "B.Cu") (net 6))
 (segment (start 26.426 23.124) (end 41.031 23.124) (width 0.25) (layer "B.Cu") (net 12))
 (segment (start 29.601 33.284) (end 32.141 35.824) (width 0.25) (layer "B.Cu") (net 4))
 (segment (start 32.141 35.824) (end 41.031 35.824) (width 0.25) (layer "B.Cu") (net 4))
 (segment (start 26.426 33.284) (end 29.601 33.284) (width 0.25) (layer "B.Cu") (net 4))
 (segment (start 26.426 28.204) (end 39.761 28.204) (width 0.25) (layer "B.Cu") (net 8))
 (segment (start 39.761 28.204) (end 41.031 29.474) (width 0.25) (layer "B.Cu") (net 8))
 (segment (start 42.301 80.909) (end 37.221 80.909) (width 0.25) (layer "B.Cu") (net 9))
 (segment (start 26.5335 73.5235) (end 34.173 81.163) (width 2) (layer "B.Cu") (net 9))
 (segment (start 34.173 81.163) (end 36.967 81.163) (width 2) (layer "B.Cu") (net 9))
 (segment (start 26.5335 66.9115) (end 26.5335 73.5235) (width 2) (layer "B.Cu") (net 9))
 (segment (start 36.967 81.163) (end 37.221 80.909) (width 2) (layer "B.Cu") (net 9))
 (segment (start 54.747 49.667) (end 54.747 65.923) (width 0.25) (layer "B.Cu") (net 5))
 (segment (start 44.841 73.289) (end 45.349 73.289) (width 2) (layer "B.Cu") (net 5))
 (segment (start 39.761 73.289) (end 44.841 73.289) (width 2) (layer "B.Cu") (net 5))
 (segment (start 50.429 68.209) (end 52.461 68.209) (width 2) (layer "B.Cu") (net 5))
 (segment (start 45.349 73.289) (end 50.429 68.209) (width 2) (layer "B.Cu") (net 5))
 (segment (start 48.006 45.974) (end 51.191 49.159) (width 0.25) (layer "B.Cu") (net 5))
 (segment (start 54.239 49.159) (end 54.747 49.667) (width 0.25) (layer "B.Cu") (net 5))
 (segment (start 51.191 49.159) (end 54.239 49.159) (width 0.25) (layer "B.Cu") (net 5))
 (segment (start 54.747 65.923) (end 52.461 68.209) (width 0.25) (layer "B.Cu") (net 5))
 (segment (start 37.221 75.829) (end 39.761 73.289) (width 2) (layer "B.Cu") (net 5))
 (segment (start 29.3745 56.7515) (end 26.5335 56.7515) (width 0.25) (layer "B.Cu") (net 2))
 (segment (start 30.871 55.255) (end 29.3745 56.7515) (width 0.25) (layer "B.Cu") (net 2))
 (segment (start 36.088 45.974) (end 30.871 51.191) (width 0.25) (layer "B.Cu") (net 2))
 (segment (start 36.088 45.974) (end 35.951 45.837) (width 0.25) (layer "B.Cu") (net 2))
 (segment (start 30.871 51.191) (end 30.871 55.255) (width 0.25) (layer "B.Cu") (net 2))
 (segment (start 35.951 45.837) (end 35.951 43.444) (width 0.25) (layer "B.Cu") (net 2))
 (segment (start 40.386 45.974) (end 36.088 45.974) (width 0.25) (layer "B.Cu") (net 2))
 (segment (start 54.747 40.777) (end 53.985 41.539) (width 0.25) (layer "B.Cu") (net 15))
 (segment (start 54.747 20.711) (end 54.747 40.777) (width 0.25) (layer "B.Cu") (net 15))
 (segment (start 53.985 41.539) (end 42.281 41.539) (width 0.25) (layer "B.Cu") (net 15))
 (segment (start 52.461 19.949) (end 53.985 19.949) (width 0.25) (layer "B.Cu") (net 15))
 (segment (start 42.281 41.539) (end 40.386 43.434) (width 0.25) (layer "B.Cu") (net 15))
 (segment (start 53.985 19.949) (end 54.747 20.711) (width 0.25) (layer "B.Cu") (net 15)))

